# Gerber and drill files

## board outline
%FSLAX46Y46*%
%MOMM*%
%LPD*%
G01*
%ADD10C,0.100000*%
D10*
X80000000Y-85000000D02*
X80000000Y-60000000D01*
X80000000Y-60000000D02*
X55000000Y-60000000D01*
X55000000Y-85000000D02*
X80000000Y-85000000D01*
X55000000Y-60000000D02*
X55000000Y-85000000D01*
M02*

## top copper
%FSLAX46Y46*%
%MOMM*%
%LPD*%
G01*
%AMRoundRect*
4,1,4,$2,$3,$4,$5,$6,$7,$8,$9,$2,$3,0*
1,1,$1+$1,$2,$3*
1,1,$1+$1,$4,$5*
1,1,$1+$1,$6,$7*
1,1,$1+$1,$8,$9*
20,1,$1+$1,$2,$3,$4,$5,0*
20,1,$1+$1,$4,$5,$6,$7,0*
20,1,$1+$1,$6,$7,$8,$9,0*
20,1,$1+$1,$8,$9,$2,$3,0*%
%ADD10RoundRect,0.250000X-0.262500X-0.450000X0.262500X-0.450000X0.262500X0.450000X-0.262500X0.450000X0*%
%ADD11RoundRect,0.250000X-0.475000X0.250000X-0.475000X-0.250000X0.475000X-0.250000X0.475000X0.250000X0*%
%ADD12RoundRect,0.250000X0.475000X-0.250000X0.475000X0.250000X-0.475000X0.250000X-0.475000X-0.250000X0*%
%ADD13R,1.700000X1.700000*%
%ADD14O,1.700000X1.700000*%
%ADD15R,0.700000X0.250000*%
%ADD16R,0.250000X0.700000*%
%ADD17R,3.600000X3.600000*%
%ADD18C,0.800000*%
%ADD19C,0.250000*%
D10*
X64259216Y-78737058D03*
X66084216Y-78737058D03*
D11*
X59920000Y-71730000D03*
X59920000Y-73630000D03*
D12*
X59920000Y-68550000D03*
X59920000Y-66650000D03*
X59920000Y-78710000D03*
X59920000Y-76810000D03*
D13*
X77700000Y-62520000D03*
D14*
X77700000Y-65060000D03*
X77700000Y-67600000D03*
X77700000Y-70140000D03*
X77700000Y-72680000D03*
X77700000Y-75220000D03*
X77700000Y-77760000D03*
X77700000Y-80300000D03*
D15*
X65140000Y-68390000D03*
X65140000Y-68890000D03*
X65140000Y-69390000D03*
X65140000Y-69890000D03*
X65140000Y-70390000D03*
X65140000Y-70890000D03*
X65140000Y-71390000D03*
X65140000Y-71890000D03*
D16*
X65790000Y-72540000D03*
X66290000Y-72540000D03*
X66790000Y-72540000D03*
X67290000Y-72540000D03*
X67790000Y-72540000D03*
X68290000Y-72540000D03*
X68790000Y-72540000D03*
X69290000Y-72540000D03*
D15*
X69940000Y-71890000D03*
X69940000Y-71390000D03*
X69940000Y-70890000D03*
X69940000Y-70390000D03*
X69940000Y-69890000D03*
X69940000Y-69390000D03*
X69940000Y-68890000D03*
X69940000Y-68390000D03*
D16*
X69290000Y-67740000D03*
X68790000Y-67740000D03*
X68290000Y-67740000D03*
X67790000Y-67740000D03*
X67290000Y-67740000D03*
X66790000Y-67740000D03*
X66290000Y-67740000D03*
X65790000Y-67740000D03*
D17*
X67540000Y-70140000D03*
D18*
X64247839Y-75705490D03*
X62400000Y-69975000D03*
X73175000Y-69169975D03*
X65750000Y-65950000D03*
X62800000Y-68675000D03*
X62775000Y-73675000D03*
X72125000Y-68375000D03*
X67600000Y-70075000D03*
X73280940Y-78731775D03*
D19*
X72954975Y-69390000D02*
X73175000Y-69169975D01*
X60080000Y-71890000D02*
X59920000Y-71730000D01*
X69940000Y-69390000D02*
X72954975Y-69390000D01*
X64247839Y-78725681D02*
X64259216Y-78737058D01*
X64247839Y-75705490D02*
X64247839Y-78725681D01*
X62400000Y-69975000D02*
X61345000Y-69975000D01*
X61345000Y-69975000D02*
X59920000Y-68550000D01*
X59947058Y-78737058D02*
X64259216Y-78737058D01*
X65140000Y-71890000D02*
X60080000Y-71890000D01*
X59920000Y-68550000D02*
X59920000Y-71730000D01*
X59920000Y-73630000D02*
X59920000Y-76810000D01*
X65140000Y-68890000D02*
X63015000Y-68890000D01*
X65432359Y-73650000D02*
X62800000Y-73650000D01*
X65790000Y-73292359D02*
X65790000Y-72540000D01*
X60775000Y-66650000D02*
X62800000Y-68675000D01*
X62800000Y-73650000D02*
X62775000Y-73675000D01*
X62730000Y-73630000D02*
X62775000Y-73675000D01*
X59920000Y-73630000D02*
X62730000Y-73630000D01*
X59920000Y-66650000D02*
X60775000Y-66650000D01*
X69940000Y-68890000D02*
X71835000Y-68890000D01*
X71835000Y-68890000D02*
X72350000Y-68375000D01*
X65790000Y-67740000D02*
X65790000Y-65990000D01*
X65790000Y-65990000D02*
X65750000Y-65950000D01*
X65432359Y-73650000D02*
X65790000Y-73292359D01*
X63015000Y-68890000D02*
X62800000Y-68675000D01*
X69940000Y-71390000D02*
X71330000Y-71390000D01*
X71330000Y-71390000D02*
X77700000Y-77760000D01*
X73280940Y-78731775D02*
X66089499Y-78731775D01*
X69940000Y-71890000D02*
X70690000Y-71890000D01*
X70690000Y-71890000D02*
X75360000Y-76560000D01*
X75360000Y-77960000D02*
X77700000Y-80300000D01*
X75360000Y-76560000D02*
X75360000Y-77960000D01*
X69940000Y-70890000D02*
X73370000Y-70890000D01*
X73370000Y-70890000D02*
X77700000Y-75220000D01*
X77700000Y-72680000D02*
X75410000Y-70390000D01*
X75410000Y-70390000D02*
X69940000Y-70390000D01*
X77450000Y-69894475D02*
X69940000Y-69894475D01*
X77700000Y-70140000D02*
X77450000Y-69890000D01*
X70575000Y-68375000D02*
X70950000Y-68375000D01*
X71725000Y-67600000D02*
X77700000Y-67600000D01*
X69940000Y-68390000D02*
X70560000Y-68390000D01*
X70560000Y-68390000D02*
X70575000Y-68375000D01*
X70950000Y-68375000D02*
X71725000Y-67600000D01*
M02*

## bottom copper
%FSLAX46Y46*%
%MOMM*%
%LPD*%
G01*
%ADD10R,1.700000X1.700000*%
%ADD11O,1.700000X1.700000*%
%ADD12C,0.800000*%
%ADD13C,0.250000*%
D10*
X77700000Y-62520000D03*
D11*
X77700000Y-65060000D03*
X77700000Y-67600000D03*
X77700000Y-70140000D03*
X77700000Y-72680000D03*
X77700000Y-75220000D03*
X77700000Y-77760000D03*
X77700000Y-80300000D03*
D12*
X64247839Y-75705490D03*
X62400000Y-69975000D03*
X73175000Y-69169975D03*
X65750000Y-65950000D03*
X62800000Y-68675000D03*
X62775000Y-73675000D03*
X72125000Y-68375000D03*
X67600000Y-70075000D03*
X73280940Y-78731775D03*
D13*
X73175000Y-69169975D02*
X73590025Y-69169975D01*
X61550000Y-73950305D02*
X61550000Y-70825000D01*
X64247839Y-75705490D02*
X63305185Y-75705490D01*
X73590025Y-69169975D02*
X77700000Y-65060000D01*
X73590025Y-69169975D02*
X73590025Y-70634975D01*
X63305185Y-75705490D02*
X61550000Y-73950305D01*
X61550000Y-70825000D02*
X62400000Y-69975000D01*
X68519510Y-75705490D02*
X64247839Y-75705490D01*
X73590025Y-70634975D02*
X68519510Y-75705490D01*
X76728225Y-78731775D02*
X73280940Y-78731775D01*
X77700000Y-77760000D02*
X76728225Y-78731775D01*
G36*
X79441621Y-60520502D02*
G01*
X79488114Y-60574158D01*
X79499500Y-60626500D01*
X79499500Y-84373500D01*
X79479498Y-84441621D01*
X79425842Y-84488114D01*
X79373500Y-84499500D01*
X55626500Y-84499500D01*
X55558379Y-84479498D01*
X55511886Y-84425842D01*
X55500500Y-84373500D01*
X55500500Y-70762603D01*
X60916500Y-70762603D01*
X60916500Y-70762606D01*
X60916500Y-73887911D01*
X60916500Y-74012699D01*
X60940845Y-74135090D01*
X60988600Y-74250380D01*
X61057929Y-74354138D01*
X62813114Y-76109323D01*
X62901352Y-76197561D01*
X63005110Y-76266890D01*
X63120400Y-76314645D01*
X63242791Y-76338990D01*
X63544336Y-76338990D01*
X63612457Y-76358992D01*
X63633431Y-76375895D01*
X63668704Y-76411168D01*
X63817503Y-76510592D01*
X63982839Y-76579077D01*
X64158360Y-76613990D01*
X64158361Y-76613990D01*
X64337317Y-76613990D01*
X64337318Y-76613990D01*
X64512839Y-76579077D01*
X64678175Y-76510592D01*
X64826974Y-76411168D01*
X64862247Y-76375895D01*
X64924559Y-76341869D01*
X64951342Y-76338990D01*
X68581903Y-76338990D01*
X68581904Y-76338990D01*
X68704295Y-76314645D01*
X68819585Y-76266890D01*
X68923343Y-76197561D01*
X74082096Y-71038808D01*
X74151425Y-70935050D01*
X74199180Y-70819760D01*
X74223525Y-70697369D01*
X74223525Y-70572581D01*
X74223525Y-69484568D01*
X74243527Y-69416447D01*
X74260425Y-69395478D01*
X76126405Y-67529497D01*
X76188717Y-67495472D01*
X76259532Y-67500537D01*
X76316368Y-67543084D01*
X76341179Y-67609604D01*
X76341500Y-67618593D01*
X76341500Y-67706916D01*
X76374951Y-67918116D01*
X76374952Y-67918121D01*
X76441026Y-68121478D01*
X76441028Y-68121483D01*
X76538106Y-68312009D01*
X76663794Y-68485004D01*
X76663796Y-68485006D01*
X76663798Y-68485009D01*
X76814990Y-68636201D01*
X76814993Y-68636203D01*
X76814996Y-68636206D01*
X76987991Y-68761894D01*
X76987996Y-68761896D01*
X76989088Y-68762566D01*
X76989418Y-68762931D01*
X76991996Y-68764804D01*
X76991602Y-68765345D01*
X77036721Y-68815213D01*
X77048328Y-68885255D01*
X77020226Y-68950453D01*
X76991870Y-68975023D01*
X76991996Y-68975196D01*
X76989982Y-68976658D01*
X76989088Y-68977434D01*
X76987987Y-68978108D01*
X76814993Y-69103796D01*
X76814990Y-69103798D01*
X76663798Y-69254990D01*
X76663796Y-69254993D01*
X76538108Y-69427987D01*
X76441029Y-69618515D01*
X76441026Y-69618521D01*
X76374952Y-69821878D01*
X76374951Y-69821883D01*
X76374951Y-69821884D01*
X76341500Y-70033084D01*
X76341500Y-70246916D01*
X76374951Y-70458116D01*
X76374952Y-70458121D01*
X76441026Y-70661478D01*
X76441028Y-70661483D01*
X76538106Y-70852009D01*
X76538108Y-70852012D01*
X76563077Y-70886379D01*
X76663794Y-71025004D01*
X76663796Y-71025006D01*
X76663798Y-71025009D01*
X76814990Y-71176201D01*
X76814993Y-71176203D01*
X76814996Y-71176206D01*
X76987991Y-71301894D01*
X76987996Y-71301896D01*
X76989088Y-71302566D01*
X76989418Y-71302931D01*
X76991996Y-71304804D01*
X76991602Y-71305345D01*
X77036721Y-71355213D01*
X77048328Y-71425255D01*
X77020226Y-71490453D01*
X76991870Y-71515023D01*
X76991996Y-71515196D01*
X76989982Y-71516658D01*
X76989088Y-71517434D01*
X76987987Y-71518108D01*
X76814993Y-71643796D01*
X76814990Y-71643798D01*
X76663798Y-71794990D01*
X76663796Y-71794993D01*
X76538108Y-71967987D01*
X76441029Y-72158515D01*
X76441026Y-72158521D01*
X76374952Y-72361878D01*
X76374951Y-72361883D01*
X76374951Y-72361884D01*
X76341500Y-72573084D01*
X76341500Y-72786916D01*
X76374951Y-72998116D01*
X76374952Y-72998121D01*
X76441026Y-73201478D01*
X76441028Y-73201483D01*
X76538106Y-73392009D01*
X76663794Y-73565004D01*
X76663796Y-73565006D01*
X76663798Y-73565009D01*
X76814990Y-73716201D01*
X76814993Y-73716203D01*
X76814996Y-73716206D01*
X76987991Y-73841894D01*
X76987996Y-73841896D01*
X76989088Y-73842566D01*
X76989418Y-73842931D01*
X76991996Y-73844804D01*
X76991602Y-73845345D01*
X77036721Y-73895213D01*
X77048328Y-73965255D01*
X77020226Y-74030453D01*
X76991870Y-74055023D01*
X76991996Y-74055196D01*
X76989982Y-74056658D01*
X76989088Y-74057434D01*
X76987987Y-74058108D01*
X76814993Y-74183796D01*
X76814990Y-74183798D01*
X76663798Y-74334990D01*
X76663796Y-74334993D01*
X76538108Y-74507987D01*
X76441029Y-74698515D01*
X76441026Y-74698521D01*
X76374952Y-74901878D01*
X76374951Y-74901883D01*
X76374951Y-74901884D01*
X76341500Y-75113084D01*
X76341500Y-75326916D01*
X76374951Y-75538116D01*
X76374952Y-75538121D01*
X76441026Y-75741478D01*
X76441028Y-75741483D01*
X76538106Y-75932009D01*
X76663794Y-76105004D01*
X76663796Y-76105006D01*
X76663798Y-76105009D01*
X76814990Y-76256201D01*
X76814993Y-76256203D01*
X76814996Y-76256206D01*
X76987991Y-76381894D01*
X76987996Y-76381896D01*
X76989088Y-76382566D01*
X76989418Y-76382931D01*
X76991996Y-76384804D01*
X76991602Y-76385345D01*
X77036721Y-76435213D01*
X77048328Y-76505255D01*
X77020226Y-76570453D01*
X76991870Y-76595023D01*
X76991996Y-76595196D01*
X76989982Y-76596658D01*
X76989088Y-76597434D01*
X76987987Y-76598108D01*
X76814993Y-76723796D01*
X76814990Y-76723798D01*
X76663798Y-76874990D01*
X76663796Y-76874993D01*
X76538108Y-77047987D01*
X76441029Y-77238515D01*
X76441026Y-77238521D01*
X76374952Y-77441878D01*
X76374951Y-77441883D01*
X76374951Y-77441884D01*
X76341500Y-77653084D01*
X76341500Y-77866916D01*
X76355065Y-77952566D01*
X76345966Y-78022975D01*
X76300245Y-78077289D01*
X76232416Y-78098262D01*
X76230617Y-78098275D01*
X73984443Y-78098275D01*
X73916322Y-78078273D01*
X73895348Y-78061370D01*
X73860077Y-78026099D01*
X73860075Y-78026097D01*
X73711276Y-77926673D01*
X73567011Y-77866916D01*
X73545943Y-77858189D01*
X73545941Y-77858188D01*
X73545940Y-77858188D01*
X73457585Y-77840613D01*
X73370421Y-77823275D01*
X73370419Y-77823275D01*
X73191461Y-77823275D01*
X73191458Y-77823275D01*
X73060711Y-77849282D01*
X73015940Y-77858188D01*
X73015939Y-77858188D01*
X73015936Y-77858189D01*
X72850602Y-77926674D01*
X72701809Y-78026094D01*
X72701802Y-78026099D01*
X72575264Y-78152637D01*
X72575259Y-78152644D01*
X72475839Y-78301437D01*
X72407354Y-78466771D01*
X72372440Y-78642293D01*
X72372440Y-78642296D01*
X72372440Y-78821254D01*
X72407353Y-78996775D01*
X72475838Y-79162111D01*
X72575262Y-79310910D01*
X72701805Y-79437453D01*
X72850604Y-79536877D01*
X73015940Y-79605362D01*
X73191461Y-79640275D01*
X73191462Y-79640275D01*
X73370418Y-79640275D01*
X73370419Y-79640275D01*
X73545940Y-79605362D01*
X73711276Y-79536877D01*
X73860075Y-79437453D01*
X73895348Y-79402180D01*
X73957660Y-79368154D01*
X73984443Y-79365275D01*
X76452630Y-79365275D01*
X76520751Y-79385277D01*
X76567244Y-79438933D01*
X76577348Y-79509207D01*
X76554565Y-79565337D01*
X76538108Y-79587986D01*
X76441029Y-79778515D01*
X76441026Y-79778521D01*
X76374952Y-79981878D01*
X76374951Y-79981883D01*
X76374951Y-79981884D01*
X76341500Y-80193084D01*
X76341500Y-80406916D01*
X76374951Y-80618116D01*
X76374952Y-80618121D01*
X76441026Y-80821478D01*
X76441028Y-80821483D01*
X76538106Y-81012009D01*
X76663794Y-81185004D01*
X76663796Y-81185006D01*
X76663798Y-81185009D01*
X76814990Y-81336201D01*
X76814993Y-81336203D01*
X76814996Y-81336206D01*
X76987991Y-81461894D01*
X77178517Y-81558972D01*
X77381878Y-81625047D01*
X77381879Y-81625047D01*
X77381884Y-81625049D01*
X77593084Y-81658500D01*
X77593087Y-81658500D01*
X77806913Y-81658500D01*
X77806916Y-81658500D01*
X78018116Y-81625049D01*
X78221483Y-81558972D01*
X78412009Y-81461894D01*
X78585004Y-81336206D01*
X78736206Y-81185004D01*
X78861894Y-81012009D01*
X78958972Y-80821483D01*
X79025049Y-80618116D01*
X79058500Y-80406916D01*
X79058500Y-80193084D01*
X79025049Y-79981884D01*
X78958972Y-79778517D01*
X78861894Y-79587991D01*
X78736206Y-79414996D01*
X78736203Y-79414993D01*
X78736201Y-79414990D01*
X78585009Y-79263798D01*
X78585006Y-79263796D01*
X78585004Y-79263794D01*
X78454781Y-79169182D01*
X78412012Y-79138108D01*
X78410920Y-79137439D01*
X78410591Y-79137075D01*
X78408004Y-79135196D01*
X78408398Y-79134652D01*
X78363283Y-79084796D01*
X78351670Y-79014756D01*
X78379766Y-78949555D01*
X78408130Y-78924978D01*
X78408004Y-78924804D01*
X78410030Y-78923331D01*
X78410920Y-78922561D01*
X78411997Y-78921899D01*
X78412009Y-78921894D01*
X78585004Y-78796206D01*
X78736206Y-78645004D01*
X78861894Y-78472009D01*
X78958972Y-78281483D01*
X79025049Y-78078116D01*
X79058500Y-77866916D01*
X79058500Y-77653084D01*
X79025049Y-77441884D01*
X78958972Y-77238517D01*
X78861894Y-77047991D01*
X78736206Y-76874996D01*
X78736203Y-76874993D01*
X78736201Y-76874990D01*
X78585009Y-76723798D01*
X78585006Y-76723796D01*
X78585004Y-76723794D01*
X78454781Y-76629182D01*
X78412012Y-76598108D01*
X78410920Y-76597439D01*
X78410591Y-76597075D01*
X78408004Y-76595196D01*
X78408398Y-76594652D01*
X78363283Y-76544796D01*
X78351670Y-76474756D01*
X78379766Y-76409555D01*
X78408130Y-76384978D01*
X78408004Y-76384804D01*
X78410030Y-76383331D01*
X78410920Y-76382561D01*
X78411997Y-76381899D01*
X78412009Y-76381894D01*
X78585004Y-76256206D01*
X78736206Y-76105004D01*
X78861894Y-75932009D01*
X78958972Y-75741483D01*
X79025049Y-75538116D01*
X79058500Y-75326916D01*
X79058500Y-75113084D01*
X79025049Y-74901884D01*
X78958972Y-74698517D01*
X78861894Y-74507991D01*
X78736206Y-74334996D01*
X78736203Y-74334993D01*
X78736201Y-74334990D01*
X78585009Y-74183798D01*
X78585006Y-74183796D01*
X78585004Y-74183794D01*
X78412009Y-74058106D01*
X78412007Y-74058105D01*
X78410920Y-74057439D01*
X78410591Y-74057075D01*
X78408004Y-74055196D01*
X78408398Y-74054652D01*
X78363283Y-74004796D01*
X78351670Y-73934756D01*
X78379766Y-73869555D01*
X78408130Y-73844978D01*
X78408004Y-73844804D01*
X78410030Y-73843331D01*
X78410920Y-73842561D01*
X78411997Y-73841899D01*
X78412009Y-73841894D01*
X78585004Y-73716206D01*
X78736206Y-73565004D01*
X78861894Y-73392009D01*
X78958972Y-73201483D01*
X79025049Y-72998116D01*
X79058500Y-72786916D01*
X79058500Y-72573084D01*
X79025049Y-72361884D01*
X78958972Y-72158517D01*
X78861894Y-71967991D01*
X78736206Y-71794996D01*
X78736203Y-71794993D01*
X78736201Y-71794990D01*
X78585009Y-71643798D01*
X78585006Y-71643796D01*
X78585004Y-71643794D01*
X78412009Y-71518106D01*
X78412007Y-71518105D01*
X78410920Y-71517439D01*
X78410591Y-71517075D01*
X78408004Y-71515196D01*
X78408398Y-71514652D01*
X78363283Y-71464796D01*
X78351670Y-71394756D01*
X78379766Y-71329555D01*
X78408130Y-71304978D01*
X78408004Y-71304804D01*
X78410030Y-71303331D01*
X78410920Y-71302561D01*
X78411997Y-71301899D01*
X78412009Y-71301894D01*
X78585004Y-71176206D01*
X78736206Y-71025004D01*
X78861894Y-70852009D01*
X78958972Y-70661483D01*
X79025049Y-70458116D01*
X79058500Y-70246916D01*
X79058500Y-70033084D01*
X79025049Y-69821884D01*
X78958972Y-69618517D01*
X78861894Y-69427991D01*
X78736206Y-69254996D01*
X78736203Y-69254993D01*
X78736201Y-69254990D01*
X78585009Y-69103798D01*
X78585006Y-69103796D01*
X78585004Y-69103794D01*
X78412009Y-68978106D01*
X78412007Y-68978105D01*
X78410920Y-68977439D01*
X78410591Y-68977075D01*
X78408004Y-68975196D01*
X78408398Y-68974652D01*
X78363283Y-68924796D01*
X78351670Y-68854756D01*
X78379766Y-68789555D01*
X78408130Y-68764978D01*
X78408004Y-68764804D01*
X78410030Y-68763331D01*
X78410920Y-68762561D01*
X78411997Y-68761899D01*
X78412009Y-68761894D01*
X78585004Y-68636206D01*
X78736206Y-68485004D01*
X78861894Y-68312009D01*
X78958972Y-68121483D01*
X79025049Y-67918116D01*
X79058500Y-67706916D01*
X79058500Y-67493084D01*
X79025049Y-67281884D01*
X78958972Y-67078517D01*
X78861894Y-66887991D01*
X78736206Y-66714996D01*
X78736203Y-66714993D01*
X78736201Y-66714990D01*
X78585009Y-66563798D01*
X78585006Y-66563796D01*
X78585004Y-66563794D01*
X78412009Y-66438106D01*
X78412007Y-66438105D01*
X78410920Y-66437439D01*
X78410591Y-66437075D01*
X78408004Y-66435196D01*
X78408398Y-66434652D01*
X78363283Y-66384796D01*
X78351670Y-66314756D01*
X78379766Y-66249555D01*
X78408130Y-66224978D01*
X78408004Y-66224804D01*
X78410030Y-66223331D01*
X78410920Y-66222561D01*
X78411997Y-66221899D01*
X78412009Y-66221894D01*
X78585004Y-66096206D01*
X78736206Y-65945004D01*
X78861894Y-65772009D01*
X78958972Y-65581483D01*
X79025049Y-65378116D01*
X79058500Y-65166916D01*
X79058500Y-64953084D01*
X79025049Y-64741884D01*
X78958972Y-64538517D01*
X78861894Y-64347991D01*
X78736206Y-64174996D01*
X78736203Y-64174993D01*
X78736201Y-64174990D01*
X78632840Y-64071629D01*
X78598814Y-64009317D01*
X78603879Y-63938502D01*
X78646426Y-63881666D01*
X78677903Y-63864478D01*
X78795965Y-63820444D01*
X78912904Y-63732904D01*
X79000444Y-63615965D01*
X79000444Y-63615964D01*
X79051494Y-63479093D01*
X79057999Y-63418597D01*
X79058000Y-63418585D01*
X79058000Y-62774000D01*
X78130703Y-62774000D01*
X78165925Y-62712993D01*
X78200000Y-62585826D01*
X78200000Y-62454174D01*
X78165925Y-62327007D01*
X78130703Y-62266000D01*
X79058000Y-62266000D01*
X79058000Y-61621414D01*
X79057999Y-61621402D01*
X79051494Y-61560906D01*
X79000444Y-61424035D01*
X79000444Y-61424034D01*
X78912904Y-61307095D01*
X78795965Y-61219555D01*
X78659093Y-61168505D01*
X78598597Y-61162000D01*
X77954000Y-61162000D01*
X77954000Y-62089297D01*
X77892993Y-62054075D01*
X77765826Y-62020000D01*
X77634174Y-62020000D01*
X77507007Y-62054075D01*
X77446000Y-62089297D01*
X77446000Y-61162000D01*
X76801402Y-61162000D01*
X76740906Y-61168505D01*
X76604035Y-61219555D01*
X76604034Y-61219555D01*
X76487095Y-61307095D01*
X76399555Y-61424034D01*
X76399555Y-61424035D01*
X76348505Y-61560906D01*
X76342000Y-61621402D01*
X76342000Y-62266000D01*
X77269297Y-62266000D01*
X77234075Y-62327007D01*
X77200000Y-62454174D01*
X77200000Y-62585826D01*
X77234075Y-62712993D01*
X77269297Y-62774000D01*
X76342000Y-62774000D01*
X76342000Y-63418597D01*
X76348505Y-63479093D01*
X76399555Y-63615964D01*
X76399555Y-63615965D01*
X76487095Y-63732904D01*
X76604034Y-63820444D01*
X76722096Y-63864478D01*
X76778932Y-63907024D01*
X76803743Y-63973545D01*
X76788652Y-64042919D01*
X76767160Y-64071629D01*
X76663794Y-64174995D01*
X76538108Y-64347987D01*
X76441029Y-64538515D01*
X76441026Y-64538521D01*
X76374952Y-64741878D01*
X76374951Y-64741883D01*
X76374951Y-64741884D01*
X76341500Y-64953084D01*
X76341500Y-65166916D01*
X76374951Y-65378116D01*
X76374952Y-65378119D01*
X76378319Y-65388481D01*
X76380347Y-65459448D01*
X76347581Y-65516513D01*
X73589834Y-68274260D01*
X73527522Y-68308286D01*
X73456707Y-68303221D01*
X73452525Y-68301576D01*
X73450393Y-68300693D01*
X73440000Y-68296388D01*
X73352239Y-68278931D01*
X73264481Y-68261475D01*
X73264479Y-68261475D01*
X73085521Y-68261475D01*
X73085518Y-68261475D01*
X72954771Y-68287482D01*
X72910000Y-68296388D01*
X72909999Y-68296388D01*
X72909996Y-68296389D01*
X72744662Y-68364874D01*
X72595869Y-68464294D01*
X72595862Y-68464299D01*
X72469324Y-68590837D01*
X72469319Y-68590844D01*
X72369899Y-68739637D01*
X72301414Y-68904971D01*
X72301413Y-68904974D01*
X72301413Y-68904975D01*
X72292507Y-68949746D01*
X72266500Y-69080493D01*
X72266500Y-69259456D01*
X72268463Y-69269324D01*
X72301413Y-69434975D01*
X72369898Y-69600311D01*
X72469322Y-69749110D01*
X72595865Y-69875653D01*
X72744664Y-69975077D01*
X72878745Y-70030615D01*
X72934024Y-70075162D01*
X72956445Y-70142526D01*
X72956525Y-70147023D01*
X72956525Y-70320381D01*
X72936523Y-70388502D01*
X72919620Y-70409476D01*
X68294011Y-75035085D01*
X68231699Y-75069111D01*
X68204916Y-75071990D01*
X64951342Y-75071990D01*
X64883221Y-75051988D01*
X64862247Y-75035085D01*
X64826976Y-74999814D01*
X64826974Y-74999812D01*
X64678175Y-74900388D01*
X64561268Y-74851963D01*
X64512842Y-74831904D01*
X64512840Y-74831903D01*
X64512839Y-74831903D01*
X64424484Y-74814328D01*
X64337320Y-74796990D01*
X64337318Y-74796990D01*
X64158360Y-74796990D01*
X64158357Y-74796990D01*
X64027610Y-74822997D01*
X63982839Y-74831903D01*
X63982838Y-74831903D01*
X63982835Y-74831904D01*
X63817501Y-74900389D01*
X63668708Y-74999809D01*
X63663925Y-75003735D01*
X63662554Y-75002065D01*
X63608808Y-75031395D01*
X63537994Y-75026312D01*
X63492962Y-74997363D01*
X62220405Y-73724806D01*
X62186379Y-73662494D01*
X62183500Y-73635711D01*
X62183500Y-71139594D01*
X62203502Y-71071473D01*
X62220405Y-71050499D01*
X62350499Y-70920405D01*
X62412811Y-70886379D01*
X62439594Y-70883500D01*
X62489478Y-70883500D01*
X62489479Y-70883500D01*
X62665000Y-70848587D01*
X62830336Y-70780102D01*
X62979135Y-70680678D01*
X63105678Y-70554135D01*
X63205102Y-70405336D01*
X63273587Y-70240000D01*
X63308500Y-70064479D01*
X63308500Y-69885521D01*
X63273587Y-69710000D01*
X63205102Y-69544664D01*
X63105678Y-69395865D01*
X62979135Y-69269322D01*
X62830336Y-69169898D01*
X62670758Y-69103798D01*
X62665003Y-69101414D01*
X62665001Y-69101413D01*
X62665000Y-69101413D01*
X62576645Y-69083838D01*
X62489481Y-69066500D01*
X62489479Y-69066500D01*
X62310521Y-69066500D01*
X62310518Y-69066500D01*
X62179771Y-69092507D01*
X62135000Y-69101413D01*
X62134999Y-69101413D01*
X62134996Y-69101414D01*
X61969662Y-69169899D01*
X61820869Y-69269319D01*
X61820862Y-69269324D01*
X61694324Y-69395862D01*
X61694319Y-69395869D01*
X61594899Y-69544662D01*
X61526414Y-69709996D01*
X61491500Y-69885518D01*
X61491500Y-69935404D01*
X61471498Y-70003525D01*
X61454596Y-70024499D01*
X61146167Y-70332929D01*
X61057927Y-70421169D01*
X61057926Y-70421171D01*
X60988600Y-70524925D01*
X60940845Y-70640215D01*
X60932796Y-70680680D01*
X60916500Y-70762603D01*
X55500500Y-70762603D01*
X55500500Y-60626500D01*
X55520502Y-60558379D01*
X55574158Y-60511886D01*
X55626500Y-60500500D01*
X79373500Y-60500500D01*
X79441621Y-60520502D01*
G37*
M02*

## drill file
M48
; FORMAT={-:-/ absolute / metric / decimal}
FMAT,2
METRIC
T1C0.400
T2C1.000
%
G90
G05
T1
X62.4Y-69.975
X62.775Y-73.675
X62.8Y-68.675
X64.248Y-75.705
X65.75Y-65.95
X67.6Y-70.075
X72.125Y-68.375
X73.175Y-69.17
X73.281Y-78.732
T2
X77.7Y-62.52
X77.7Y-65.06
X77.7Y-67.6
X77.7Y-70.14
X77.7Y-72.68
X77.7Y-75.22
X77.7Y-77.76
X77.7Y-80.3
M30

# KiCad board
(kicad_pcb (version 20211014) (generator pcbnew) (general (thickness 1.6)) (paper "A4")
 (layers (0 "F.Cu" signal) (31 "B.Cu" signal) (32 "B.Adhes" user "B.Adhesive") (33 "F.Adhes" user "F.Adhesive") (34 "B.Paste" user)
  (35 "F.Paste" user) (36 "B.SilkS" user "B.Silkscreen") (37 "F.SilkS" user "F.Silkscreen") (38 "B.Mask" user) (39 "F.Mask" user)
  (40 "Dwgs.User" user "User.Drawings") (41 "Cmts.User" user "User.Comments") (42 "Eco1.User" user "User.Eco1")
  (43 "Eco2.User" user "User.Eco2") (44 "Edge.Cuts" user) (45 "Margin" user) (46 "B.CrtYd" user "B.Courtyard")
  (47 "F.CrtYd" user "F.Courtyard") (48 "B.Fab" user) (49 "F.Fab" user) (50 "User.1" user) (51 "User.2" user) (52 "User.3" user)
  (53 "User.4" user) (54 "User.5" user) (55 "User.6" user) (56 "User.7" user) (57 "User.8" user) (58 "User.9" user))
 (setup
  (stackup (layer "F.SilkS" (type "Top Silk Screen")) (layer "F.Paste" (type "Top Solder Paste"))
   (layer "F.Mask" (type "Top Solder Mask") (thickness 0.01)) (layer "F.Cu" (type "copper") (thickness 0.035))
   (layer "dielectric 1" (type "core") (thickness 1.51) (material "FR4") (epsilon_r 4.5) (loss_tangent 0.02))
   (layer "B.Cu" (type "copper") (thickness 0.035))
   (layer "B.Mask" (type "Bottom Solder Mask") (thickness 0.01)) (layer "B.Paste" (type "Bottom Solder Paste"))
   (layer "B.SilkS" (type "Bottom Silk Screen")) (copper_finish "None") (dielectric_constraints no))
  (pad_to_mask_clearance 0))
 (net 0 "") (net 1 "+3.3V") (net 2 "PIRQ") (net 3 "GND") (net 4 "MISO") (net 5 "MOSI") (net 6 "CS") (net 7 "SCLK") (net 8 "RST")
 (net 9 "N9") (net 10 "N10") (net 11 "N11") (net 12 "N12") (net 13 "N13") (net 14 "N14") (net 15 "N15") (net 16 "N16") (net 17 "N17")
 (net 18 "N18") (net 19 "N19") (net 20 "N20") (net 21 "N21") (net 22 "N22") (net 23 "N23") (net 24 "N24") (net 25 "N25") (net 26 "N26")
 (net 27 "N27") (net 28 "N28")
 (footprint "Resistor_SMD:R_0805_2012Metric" (layer "F.Cu") (at 65.171716 78.737058)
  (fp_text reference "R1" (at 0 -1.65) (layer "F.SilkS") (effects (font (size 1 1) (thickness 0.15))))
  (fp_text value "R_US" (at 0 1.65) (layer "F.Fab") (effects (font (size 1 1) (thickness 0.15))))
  (pad "1" smd roundrect (at -0.9125 0) (size 1.025 1.4) (layers "F.Cu" "F.Paste" "F.Mask") (roundrect_rratio 0.243902439) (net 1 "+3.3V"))
  (pad "2" smd roundrect (at 0.9125 0) (size 1.025 1.4) (layers "F.Cu" "F.Paste" "F.Mask") (roundrect_rratio 0.243902439) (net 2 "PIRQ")))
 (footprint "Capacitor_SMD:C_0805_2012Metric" (layer "F.Cu") (at 59.92 72.68 -90)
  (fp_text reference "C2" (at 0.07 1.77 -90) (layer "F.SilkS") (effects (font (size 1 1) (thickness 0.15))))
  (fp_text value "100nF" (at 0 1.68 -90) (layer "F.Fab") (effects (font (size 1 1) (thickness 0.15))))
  (pad "1" smd roundrect (at -0.95 0 270) (size 1 1.45) (layers "F.Cu" "F.Paste" "F.Mask") (roundrect_rratio 0.25) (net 1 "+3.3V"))
  (pad "2" smd roundrect (at 0.95 0 270) (size 1 1.45) (layers "F.Cu" "F.Paste" "F.Mask") (roundrect_rratio 0.25) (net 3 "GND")))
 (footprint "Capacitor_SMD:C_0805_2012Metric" (layer "F.Cu") (at 59.92 67.6 90)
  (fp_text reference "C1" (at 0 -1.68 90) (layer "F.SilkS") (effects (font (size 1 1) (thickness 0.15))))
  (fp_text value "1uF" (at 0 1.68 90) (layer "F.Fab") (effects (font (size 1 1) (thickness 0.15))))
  (pad "1" smd roundrect (at -0.95 0 90) (size 1 1.45) (layers "F.Cu" "F.Paste" "F.Mask") (roundrect_rratio 0.25) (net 1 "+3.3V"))
  (pad "2" smd roundrect (at 0.95 0 90) (size 1 1.45) (layers "F.Cu" "F.Paste" "F.Mask") (roundrect_rratio 0.25) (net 3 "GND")))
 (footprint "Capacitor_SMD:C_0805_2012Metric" (layer "F.Cu") (at 59.92 77.76 90)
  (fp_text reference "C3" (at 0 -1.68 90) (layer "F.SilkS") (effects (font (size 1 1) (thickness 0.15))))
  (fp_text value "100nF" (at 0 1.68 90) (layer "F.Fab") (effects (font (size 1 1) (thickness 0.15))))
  (pad "1" smd roundrect (at -0.95 0 90) (size 1 1.45) (layers "F.Cu" "F.Paste" "F.Mask") (roundrect_rratio 0.25) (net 1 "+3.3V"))
  (pad "2" smd roundrect (at 0.95 0 90) (size 1 1.45) (layers "F.Cu" "F.Paste" "F.Mask") (roundrect_rratio 0.25) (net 3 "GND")))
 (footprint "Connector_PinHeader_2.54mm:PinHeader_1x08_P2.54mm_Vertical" (layer "F.Cu") (at 77.7 62.52)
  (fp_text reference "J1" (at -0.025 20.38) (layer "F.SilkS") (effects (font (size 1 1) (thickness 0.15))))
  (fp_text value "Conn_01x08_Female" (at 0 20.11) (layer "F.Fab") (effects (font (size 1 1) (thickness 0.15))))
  (pad "1" thru_hole rect (at 0 0) (size 1.7 1.7) (drill 1) (layers *.Cu *.Mask) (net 3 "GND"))
  (pad "2" thru_hole oval (at 0 2.54) (size 1.7 1.7) (drill 1) (layers *.Cu *.Mask) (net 1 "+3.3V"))
  (pad "3" thru_hole oval (at 0 5.08) (size 1.7 1.7) (drill 1) (layers *.Cu *.Mask) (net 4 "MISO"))
  (pad "4" thru_hole oval (at 0 7.62) (size 1.7 1.7) (drill 1) (layers *.Cu *.Mask) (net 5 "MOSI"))
  (pad "5" thru_hole oval (at 0 10.16) (size 1.7 1.7) (drill 1) (layers *.Cu *.Mask) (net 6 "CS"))
  (pad "6" thru_hole oval (at 0 12.7) (size 1.7 1.7) (drill 1) (layers *.Cu *.Mask) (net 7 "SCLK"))
  (pad "7" thru_hole oval (at 0 15.24) (size 1.7 1.7) (drill 1) (layers *.Cu *.Mask) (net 2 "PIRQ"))
  (pad "8" thru_hole oval (at 0 17.78) (size 1.7 1.7) (drill 1) (layers *.Cu *.Mask) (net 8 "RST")))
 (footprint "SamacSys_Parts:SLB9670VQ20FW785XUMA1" (layer "F.Cu") (at 67.54 70.14)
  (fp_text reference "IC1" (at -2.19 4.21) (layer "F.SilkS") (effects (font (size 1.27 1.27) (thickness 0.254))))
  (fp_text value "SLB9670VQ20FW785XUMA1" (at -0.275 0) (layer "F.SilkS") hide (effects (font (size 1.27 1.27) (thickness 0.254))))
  (pad "1" smd rect locked (at -2.4 -1.75 90) (size 0.25 0.7) (layers "F.Cu" "F.Paste" "F.Mask") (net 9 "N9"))
  (pad "2" smd rect locked (at -2.4 -1.25 90) (size 0.25 0.7) (layers "F.Cu" "F.Paste" "F.Mask") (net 3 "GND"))
  (pad "3" smd rect locked (at -2.4 -0.75 90) (size 0.25 0.7) (layers "F.Cu" "F.Paste" "F.Mask") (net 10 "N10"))
  (pad "4" smd rect locked (at -2.4 -0.25 90) (size 0.25 0.7) (layers "F.Cu" "F.Paste" "F.Mask") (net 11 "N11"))
  (pad "5" smd rect locked (at -2.4 0.25 90) (size 0.25 0.7) (layers "F.Cu" "F.Paste" "F.Mask") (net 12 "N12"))
  (pad "6" smd rect locked (at -2.4 0.75 90) (size 0.25 0.7) (layers "F.Cu" "F.Paste" "F.Mask") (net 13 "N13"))
  (pad "7" smd rect locked (at -2.4 1.25 90) (size 0.25 0.7) (layers "F.Cu" "F.Paste" "F.Mask") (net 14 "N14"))
  (pad "8" smd rect locked (at -2.4 1.75 90) (size 0.25 0.7) (layers "F.Cu" "F.Paste" "F.Mask") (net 1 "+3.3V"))
  (pad "9" smd rect locked (at -1.75 2.4) (size 0.25 0.7) (layers "F.Cu" "F.Paste" "F.Mask") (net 3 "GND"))
  (pad "10" smd rect locked (at -1.25 2.4) (size 0.25 0.7) (layers "F.Cu" "F.Paste" "F.Mask") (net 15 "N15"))
  (pad "11" smd rect locked (at -0.75 2.4) (size 0.25 0.7) (layers "F.Cu" "F.Paste" "F.Mask") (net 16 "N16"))
  (pad "12" smd rect locked (at -0.25 2.4) (size 0.25 0.7) (layers "F.Cu" "F.Paste" "F.Mask") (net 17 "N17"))
  (pad "13" smd rect locked (at 0.25 2.4) (size 0.25 0.7) (layers "F.Cu" "F.Paste" "F.Mask") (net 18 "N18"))
  (pad "14" smd rect locked (at 0.75 2.4) (size 0.25 0.7) (layers "F.Cu" "F.Paste" "F.Mask") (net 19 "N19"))
  (pad "15" smd rect locked (at 1.25 2.4) (size 0.25 0.7) (layers "F.Cu" "F.Paste" "F.Mask") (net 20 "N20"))
  (pad "16" smd rect locked (at 1.75 2.4) (size 0.25 0.7) (layers "F.Cu" "F.Paste" "F.Mask") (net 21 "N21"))
  (pad "17" smd rect locked (at 2.4 1.75 90) (size 0.25 0.7) (layers "F.Cu" "F.Paste" "F.Mask") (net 8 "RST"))
  (pad "18" smd rect locked (at 2.4 1.25 90) (size 0.25 0.7) (layers "F.Cu" "F.Paste" "F.Mask") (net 2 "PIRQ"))
  (pad "19" smd rect locked (at 2.4 0.75 90) (size 0.25 0.7) (layers "F.Cu" "F.Paste" "F.Mask") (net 7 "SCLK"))
  (pad "20" smd rect locked (at 2.4 0.25 90) (size 0.25 0.7) (layers "F.Cu" "F.Paste" "F.Mask") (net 6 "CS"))
  (pad "21" smd rect locked (at 2.4 -0.25 90) (size 0.25 0.7) (layers "F.Cu" "F.Paste" "F.Mask") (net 5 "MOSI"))
  (pad "22" smd rect locked (at 2.4 -0.75 90) (size 0.25 0.7) (layers "F.Cu" "F.Paste" "F.Mask") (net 1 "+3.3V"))
  (pad "23" smd rect locked (at 2.4 -1.25 90) (size 0.25 0.7) (layers "F.Cu" "F.Paste" "F.Mask") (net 3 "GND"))
  (pad "24" smd rect locked (at 2.4 -1.75 90) (size 0.25 0.7) (layers "F.Cu" "F.Paste" "F.Mask") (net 4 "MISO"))
  (pad "25" smd rect locked (at 1.75 -2.4) (size 0.25 0.7) (layers "F.Cu" "F.Paste" "F.Mask") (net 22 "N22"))
  (pad "26" smd rect locked (at 1.25 -2.4) (size 0.25 0.7) (layers "F.Cu" "F.Paste" "F.Mask") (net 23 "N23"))
  (pad "27" smd rect locked (at 0.75 -2.4) (size 0.25 0.7) (layers "F.Cu" "F.Paste" "F.Mask") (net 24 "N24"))
  (pad "28" smd rect locked (at 0.25 -2.4) (size 0.25 0.7) (layers "F.Cu" "F.Paste" "F.Mask") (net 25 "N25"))
  (pad "29" smd rect locked (at -0.25 -2.4) (size 0.25 0.7) (layers "F.Cu" "F.Paste" "F.Mask") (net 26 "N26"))
  (pad "30" smd rect locked (at -0.75 -2.4) (size 0.25 0.7) (layers "F.Cu" "F.Paste" "F.Mask") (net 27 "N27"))
  (pad "31" smd rect locked (at -1.25 -2.4) (size 0.25 0.7) (layers "F.Cu" "F.Paste" "F.Mask") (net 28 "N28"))
  (pad "32" smd rect locked (at -1.75 -2.4) (size 0.25 0.7) (layers "F.Cu" "F.Paste" "F.Mask") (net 3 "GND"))
  (pad "33" smd rect locked (at 0 0) (size 3.6 3.6) (layers "F.Cu" "F.Paste" "F.Mask") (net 3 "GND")))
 (gr_line (start 80 85) (end 80 60) (layer "Edge.Cuts") (width 0.1))
 (gr_line (start 80 60) (end 55 60) (layer "Edge.Cuts") (width 0.1))
 (gr_line (start 55 85) (end 80 85) (layer "Edge.Cuts") (width 0.1))
 (gr_line (start 55 60) (end 55 85) (layer "Edge.Cuts") (width 0.1))
 (segment (start 72.954975 69.39) (end 73.175 69.169975) (width 0.25) (layer "F.Cu") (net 1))
 (segment (start 60.08 71.89) (end 59.92 71.73) (width 0.25) (layer "F.Cu") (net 1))
 (segment (start 69.94 69.39) (end 72.954975 69.39) (width 0.25) (layer "F.Cu") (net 1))
 (segment (start 64.247839 78.725681) (end 64.259216 78.737058) (width 0.25) (layer "F.Cu") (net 1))
 (segment (start 64.247839 75.70549) (end 64.247839 78.725681) (width 0.25) (layer "F.Cu") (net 1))
 (segment (start 62.4 69.975) (end 61.345 69.975) (width 0.25) (layer "F.Cu") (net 1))
 (segment (start 61.345 69.975) (end 59.92 68.55) (width 0.25) (layer "F.Cu") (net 1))
 (segment (start 59.947058 78.737058) (end 64.259216 78.737058) (width 0.25) (layer "F.Cu") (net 1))
 (segment (start 65.14 71.89) (end 60.08 71.89) (width 0.25) (layer "F.Cu") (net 1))
 (segment (start 59.92 68.55) (end 59.92 71.73) (width 0.25) (layer "F.Cu") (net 1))
 (via (at 64.247839 75.70549) (size 0.8) (drill 0.4) (layers "F.Cu" "B.Cu") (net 1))
 (via (at 62.4 69.975) (size 0.8) (drill 0.4) (layers "F.Cu" "B.Cu") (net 1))
 (via (at 73.175 69.169975) (size 0.8) (drill 0.4) (layers "F.Cu" "B.Cu") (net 1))
 (segment (start 73.175 69.169975) (end 73.590025 69.169975) (width 0.25) (layer "B.Cu") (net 1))
 (segment (start 61.55 73.950305) (end 61.55 70.825) (width 0.25) (layer "B.Cu") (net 1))
 (segment (start 64.247839 75.70549) (end 63.305185 75.70549) (width 0.25) (layer "B.Cu") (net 1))
 (segment (start 73.590025 69.169975) (end 77.7 65.06) (width 0.25) (layer "B.Cu") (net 1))
 (segment (start 73.590025 69.169975) (end 73.590025 70.634975) (width 0.25) (layer "B.Cu") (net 1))
 (segment (start 63.305185 75.70549) (end 61.55 73.950305) (width 0.25) (layer "B.Cu") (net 1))
 (segment (start 61.55 70.825) (end 62.4 69.975) (width 0.25) (layer "B.Cu") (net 1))
 (segment (start 68.51951 75.70549) (end 64.247839 75.70549) (width 0.25) (layer "B.Cu") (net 1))
 (segment (start 73.590025 70.634975) (end 68.51951 75.70549) (width 0.25) (layer "B.Cu") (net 1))
 (segment (start 59.92 73.63) (end 59.92 76.81) (width 0.25) (layer "F.Cu") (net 3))
 (segment (start 65.14 68.89) (end 63.015 68.89) (width 0.25) (layer "F.Cu") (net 3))
 (segment (start 65.432359 73.65) (end 62.8 73.65) (width 0.25) (layer "F.Cu") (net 3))
 (segment (start 65.79 73.292359) (end 65.79 72.54) (width 0.25) (layer "F.Cu") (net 3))
 (segment (start 60.775 66.65) (end 62.8 68.675) (width 0.25) (layer "F.Cu") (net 3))
 (segment (start 62.8 73.65) (end 62.775 73.675) (width 0.25) (layer "F.Cu") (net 3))
 (segment (start 62.73 73.63) (end 62.775 73.675) (width 0.25) (layer "F.Cu") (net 3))
 (segment (start 59.92 73.63) (end 62.73 73.63) (width 0.25) (layer "F.Cu") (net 3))
 (segment (start 59.92 66.65) (end 60.775 66.65) (width 0.25) (layer "F.Cu") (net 3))
 (segment (start 69.94 68.89) (end 71.835 68.89) (width 0.25) (layer "F.Cu") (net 3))
 (segment (start 71.835 68.89) (end 72.35 68.375) (width 0.25) (layer "F.Cu") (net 3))
 (segment (start 65.79 67.74) (end 65.79 65.99) (width 0.25) (layer "F.Cu") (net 3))
 (segment (start 65.79 65.99) (end 65.75 65.95) (width 0.25) (layer "F.Cu") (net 3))
 (segment (start 65.432359 73.65) (end 65.79 73.292359) (width 0.25) (layer "F.Cu") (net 3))
 (segment (start 63.015 68.89) (end 62.8 68.675) (width 0.25) (layer "F.Cu") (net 3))
 (via (at 65.75 65.95) (size 0.8) (drill 0.4) (layers "F.Cu" "B.Cu") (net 3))
 (via (at 62.8 68.675) (size 0.8) (drill 0.4) (layers "F.Cu" "B.Cu") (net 3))
 (via (at 62.775 73.675) (size 0.8) (drill 0.4) (layers "F.Cu" "B.Cu") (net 3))
 (via (at 72.125 68.375) (size 0.8) (drill 0.4) (layers "F.Cu" "B.Cu") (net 3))
 (via (at 67.6 70.075) (size 0.8) (drill 0.4) (layers "F.Cu" "B.Cu") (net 3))
 (segment (start 69.94 71.39) (end 71.33 71.39) (width 0.25) (layer "F.Cu") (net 2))
 (segment (start 71.33 71.39) (end 77.7 77.76) (width 0.25) (layer "F.Cu") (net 2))
 (segment (start 73.28094 78.731775) (end 66.089499 78.731775) (width 0.25) (layer "F.Cu") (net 2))
 (via (at 73.28094 78.731775) (size 0.8) (drill 0.4) (layers "F.Cu" "B.Cu") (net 2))
 (segment (start 76.728225 78.731775) (end 73.28094 78.731775) (width 0.25) (layer "B.Cu") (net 2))
 (segment (start 77.7 77.76) (end 76.728225 78.731775) (width 0.25) (layer "B.Cu") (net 2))
 (segment (start 69.94 71.89) (end 70.69 71.89) (width 0.25) (layer "F.Cu") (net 8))
 (segment (start 70.69 71.89) (end 75.36 76.56) (width 0.25) (layer "F.Cu") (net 8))
 (segment (start 75.36 77.96) (end 77.7 80.3) (width 0.25) (layer "F.Cu") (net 8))
 (segment (start 75.36 76.56) (end 75.36 77.96) (width 0.25) (layer "F.Cu") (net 8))
 (segment (start 69.94 70.89) (end 73.37 70.89) (width 0.25) (layer "F.Cu") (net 7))
 (segment (start 73.37 70.89) (end 77.7 75.22) (width 0.25) (layer "F.Cu") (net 7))
 (segment (start 77.7 72.68) (end 75.41 70.39) (width 0.25) (layer "F.Cu") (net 6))
 (segment (start 75.41 70.39) (end 69.94 70.39) (width 0.25) (layer "F.Cu") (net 6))
 (segment (start 77.45 69.894475) (end 69.94 69.894475) (width 0.25) (layer "F.Cu") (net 5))
 (segment (start 77.7 70.14) (end 77.45 69.89) (width 0.25) (layer "F.Cu") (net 5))
 (segment (start 70.575 68.375) (end 70.95 68.375) (width 0.25) (layer "F.Cu") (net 4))
 (segment (start 71.725 67.6) (end 77.7 67.6) (width 0.25) (layer "F.Cu") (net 4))
 (segment (start 69.94 68.39) (end 70.56 68.39) (width 0.25) (layer "F.Cu") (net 4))
 (segment (start 70.56 68.39) (end 70.575 68.375) (width 0.25) (layer "F.Cu") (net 4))
 (segment (start 70.95 68.375) (end 71.725 67.6) (width 0.25) (layer "F.Cu") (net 4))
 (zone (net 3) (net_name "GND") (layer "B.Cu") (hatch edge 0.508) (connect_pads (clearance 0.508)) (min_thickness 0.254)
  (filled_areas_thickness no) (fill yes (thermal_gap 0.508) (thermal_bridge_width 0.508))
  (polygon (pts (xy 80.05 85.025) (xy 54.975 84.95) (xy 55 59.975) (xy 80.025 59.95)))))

